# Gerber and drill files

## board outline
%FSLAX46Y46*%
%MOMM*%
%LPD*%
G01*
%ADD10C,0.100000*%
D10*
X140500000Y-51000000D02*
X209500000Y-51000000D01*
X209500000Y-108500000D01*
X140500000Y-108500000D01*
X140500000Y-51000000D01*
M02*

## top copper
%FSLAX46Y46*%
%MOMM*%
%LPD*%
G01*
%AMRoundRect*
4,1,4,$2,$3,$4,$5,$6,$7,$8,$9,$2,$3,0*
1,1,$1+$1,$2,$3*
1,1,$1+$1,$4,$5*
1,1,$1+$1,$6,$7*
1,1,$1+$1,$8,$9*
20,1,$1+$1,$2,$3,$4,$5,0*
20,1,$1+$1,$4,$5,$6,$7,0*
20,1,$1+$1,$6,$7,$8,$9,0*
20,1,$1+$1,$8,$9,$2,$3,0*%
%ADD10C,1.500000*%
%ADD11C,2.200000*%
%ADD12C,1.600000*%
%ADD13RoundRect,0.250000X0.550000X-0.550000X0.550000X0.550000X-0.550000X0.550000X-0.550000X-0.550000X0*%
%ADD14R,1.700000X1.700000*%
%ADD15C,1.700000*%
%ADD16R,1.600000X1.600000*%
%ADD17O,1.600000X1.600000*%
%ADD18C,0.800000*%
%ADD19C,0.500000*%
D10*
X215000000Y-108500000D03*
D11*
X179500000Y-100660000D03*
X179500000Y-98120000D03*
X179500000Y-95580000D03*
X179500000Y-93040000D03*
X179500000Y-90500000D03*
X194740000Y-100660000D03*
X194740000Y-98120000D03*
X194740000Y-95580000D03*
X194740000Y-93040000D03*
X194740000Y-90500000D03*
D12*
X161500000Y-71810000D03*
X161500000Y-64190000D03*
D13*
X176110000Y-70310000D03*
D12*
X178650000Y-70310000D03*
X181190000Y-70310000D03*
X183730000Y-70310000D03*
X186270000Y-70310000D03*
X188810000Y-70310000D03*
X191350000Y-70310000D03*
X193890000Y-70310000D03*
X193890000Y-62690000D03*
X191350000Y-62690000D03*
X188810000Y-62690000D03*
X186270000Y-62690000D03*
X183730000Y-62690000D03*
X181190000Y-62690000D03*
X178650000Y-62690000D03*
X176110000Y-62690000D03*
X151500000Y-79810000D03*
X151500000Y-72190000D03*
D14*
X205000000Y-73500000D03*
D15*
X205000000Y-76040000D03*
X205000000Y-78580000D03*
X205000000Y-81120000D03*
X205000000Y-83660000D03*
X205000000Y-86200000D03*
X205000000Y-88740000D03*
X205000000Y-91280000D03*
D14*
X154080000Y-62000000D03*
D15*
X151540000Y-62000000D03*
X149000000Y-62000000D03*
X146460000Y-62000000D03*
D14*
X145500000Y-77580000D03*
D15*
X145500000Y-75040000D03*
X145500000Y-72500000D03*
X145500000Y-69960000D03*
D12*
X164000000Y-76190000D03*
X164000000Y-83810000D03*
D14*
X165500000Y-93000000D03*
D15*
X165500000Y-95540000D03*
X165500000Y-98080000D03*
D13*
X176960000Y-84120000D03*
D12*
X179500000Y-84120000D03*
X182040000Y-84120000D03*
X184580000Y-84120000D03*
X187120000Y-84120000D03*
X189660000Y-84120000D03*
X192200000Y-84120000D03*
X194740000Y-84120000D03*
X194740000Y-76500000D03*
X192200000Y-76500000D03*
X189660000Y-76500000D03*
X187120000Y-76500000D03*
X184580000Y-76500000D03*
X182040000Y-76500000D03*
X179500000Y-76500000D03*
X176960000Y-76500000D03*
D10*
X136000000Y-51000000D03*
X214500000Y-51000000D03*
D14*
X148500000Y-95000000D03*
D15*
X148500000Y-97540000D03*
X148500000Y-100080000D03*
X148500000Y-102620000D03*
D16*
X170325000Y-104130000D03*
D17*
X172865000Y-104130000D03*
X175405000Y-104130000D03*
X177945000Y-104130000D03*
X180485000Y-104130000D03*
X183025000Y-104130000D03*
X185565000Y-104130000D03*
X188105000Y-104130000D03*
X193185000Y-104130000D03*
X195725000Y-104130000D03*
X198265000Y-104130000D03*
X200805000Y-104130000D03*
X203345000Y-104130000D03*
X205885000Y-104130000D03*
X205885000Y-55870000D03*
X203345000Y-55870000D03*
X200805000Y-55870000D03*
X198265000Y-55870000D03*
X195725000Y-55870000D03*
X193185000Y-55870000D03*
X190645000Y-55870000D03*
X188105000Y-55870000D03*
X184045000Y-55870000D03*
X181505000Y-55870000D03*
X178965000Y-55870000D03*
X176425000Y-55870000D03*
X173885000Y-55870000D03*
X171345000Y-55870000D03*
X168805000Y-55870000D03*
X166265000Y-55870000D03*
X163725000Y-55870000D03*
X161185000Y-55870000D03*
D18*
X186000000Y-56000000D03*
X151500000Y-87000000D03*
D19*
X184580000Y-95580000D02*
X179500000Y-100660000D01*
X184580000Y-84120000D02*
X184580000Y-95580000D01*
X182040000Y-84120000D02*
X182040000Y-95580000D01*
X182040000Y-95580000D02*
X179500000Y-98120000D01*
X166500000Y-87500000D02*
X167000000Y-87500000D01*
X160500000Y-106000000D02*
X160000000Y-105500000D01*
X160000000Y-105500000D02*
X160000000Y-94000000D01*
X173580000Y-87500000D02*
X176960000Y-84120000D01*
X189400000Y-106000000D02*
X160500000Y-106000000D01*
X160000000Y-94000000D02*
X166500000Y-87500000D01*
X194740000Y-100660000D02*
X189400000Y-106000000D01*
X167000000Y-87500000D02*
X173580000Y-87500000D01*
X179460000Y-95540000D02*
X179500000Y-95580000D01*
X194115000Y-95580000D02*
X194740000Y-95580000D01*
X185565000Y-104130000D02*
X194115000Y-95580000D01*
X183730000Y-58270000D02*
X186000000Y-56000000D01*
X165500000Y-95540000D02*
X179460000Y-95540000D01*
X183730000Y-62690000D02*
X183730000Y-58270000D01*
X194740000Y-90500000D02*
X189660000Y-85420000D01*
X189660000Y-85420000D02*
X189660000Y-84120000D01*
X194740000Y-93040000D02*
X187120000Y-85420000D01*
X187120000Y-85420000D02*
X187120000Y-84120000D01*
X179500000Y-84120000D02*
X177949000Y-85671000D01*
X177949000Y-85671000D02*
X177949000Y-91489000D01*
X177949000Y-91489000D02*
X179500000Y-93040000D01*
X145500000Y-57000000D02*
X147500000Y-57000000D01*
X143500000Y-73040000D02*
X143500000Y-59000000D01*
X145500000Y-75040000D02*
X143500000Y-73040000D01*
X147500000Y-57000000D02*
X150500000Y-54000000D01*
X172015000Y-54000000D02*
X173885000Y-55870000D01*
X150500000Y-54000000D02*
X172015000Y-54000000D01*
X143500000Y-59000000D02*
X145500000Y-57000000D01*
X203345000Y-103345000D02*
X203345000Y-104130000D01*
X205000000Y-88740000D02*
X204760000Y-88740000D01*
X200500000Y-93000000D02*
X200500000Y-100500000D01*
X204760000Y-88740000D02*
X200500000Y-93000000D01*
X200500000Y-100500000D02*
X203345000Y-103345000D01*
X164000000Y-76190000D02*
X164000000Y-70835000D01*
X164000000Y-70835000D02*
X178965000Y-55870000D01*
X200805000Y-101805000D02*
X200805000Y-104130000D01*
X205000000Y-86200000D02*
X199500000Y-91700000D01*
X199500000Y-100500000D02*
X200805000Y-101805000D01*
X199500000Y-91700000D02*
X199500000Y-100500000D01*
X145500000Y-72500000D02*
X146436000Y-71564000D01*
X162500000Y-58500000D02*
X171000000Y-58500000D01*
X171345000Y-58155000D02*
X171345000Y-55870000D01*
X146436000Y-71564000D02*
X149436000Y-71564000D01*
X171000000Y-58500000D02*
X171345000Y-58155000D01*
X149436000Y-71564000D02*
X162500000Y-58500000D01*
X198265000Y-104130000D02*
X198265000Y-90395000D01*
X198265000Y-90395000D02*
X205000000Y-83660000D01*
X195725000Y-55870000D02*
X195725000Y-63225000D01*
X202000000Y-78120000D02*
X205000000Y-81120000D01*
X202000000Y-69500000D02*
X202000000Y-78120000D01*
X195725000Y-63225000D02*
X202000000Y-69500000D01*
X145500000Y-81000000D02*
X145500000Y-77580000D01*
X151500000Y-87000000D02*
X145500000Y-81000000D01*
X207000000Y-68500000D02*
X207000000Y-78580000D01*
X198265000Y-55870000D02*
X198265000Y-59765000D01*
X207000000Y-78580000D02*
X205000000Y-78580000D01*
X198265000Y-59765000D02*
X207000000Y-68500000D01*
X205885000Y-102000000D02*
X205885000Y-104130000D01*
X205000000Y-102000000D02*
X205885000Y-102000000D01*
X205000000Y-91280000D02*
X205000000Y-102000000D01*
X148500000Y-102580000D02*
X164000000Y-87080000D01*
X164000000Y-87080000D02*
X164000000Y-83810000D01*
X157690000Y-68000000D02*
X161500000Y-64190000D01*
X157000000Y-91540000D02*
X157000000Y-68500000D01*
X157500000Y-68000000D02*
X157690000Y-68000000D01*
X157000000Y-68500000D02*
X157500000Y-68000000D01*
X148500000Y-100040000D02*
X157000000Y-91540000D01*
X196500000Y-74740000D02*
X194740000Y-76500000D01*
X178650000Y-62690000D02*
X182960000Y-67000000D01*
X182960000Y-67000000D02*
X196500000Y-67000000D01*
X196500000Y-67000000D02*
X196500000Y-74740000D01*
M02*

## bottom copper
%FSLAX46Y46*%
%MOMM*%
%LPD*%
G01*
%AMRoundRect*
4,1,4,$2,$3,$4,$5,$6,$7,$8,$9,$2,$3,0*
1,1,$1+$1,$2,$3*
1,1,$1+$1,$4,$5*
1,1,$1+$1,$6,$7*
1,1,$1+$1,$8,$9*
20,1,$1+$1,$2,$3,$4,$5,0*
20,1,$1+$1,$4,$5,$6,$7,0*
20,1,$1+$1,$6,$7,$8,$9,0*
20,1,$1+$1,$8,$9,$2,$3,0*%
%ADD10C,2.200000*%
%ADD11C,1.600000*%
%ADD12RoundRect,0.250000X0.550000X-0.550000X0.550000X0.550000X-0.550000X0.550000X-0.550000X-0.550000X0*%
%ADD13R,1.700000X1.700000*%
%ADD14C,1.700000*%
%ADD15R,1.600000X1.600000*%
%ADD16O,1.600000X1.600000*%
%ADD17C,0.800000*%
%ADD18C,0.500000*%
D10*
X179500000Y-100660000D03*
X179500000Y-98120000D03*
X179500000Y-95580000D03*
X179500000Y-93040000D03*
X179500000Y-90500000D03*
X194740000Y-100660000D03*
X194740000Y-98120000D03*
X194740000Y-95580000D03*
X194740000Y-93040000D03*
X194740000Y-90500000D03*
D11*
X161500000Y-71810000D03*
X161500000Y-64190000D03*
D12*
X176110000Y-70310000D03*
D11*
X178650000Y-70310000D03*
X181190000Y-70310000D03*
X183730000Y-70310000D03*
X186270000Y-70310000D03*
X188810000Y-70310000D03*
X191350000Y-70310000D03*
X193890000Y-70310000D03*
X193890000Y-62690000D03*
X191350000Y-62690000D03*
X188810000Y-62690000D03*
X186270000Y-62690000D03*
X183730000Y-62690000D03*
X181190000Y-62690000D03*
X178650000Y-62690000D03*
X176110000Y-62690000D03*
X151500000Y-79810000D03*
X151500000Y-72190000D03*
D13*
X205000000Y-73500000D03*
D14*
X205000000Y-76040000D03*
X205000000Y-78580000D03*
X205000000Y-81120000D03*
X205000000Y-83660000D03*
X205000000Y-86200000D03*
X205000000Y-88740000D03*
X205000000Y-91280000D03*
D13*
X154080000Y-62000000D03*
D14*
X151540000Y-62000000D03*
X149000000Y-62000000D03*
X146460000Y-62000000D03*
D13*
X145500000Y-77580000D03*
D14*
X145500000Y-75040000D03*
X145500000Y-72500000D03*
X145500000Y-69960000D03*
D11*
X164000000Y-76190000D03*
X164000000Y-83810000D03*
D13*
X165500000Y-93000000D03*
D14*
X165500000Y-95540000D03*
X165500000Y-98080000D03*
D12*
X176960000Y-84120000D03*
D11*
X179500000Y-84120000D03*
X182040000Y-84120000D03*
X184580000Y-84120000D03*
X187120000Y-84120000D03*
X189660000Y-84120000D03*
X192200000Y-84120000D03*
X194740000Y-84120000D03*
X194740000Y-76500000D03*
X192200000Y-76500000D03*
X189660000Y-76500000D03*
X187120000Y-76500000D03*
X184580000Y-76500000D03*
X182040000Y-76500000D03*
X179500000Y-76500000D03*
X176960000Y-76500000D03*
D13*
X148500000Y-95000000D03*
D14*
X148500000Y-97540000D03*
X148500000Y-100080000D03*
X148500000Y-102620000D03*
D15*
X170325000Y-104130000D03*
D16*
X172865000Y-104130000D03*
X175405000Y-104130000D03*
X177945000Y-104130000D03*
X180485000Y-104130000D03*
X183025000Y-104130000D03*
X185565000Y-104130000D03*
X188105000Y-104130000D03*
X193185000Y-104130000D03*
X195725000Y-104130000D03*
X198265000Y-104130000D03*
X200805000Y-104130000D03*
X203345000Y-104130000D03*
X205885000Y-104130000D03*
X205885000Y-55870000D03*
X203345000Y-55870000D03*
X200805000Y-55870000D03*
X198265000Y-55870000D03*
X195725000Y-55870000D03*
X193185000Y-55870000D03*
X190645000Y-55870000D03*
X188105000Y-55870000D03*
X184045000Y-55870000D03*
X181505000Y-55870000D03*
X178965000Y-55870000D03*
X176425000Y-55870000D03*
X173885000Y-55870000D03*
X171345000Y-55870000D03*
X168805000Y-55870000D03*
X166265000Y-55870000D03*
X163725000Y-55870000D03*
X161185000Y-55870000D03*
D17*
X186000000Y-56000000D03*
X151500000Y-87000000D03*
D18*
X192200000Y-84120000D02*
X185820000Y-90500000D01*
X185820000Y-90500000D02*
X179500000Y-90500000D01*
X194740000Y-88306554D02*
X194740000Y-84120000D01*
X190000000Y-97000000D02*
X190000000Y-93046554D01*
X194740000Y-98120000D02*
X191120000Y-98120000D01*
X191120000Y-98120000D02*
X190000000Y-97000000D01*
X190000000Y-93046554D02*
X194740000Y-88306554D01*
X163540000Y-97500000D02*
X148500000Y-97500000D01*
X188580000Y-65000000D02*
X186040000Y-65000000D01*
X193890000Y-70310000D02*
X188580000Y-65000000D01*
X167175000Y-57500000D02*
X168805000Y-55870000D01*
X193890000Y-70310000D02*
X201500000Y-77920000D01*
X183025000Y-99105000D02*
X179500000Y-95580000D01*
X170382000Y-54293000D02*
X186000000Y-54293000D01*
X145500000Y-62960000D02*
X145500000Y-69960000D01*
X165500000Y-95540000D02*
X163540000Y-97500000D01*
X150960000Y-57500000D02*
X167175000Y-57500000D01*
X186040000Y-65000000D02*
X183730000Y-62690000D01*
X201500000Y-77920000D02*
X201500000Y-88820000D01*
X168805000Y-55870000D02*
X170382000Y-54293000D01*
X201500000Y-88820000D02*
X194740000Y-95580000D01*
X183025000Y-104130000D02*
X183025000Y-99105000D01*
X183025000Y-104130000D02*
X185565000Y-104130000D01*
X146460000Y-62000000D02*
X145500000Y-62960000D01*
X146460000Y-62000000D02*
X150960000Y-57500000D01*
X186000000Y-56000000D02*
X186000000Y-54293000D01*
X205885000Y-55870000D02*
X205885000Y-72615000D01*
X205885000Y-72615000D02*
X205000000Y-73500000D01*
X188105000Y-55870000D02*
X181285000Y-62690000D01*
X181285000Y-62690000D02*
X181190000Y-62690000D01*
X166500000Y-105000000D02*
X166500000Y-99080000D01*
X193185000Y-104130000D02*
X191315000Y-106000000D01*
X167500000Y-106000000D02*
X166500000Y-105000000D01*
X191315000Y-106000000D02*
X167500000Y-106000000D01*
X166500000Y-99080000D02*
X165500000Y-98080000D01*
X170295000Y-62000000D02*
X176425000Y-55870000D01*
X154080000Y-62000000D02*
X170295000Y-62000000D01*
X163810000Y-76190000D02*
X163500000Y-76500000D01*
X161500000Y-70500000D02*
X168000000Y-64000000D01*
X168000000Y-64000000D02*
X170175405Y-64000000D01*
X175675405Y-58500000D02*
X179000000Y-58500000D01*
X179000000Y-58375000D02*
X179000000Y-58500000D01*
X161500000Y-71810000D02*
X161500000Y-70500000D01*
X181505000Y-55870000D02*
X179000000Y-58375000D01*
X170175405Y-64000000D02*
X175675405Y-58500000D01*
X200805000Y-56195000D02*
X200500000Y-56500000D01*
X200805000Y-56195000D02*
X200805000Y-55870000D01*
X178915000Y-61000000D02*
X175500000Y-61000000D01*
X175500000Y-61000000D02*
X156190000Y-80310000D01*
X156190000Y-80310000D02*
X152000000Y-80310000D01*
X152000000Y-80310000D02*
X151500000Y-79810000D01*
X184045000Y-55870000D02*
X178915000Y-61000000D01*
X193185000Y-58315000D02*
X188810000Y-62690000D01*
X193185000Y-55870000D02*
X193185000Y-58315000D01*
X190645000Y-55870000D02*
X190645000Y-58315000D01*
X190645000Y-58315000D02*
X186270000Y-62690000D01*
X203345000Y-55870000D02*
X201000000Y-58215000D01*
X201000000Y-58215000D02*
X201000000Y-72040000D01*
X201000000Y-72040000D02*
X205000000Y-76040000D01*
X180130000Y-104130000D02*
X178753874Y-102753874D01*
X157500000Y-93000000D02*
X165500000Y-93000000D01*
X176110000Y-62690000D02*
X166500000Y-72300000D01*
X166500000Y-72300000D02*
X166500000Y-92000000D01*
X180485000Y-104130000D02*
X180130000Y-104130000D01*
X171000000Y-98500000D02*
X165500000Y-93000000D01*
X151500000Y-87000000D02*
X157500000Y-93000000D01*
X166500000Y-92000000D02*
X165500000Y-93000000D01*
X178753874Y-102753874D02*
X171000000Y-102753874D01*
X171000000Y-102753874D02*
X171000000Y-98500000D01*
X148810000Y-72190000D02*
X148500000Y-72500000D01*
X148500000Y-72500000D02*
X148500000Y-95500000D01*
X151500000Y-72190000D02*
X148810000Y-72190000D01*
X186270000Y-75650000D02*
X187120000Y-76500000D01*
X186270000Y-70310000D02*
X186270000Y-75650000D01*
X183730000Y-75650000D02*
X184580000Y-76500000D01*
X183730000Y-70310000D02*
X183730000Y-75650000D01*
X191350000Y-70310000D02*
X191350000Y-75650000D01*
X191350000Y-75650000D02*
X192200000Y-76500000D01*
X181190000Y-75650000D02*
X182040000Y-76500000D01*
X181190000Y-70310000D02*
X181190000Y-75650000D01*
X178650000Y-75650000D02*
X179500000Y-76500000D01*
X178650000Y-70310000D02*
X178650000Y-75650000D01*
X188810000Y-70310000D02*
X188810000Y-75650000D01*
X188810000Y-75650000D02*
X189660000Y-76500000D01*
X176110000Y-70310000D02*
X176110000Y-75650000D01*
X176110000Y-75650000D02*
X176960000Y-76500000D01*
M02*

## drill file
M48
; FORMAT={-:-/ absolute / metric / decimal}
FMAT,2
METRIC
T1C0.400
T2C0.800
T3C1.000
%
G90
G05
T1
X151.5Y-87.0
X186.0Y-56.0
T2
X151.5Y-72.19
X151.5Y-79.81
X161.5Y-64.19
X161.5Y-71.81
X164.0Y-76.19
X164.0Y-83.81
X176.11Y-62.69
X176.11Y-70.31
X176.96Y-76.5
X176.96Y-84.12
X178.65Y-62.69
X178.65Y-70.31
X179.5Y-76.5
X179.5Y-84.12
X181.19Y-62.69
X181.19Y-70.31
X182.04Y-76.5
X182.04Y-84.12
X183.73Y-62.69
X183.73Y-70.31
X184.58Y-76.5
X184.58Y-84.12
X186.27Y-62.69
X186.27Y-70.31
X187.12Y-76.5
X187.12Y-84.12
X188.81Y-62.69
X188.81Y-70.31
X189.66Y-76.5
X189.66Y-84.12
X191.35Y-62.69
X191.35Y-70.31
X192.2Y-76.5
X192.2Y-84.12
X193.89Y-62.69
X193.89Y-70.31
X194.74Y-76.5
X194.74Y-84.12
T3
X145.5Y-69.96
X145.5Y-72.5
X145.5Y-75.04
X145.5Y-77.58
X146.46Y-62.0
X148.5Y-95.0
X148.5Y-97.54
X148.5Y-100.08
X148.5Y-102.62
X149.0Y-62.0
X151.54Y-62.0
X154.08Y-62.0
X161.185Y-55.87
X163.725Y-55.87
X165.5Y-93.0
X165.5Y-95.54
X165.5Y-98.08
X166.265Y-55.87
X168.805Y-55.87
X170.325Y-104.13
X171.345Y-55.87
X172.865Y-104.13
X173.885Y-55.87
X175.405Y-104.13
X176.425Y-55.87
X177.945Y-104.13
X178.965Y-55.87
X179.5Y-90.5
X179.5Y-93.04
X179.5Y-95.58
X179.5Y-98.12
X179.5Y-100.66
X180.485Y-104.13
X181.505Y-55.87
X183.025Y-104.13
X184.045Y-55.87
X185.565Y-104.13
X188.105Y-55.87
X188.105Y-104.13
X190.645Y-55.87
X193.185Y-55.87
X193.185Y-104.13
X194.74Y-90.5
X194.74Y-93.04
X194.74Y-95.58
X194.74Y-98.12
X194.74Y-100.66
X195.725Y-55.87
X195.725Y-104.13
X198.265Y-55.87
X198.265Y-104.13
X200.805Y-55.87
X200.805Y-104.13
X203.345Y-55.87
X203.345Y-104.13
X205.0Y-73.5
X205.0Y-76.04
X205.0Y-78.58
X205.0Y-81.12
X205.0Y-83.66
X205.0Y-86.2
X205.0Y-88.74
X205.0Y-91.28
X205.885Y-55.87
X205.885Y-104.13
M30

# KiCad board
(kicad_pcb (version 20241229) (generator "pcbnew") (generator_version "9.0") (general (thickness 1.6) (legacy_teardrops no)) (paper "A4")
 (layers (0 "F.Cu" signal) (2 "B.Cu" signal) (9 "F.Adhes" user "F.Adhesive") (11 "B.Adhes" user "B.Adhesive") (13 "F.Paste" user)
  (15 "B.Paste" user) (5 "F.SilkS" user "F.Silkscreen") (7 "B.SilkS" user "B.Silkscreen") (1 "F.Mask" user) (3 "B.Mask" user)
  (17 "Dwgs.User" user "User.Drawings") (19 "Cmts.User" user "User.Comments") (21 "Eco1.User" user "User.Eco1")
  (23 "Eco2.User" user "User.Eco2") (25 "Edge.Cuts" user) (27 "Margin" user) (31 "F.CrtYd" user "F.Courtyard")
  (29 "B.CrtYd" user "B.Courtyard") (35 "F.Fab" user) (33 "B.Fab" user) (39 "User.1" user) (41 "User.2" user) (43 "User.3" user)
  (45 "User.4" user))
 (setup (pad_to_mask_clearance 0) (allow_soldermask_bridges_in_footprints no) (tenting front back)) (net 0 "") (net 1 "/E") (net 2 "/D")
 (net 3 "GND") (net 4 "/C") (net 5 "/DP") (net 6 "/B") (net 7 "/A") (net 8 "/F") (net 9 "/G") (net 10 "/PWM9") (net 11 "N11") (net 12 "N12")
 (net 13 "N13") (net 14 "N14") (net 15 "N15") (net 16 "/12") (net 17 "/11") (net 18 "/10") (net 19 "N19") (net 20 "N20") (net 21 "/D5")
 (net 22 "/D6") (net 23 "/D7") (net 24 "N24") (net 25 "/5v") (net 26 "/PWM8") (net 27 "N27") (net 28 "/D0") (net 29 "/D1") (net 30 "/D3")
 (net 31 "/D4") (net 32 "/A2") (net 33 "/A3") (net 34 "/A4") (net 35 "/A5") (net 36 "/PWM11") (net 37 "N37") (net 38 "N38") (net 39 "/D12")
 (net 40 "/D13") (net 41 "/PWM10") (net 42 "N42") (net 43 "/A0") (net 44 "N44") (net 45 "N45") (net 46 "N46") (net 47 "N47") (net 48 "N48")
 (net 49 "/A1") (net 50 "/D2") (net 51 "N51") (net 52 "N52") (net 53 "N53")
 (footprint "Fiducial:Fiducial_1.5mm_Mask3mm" (layer "F.Cu") (at 215 108.5)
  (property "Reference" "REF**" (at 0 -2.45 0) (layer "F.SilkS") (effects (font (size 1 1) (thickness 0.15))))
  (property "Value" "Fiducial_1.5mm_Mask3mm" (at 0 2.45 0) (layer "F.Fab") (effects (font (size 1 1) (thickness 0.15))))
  (pad "" smd circle (at 0 0) (size 1.5 1.5) (layers "F.Cu" "F.Mask") (solder_mask_margin 0.75)))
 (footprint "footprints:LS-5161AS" (layer "F.Cu") (at 179.5 100.66 90)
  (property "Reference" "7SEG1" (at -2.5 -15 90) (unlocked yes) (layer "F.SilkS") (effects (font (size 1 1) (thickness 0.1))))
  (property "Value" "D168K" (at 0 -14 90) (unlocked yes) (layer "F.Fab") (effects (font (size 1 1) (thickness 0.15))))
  (pad "1" thru_hole circle (at 0 0 90) (size 2.2 2.2) (drill 1) (layers "*.Cu" "*.Mask") (remove_unused_layers no) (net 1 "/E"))
  (pad "2" thru_hole circle (at 2.54 0 90) (size 2.2 2.2) (drill 1) (layers "*.Cu" "*.Mask") (remove_unused_layers no) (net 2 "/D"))
  (pad "3" thru_hole circle (at 5.08 0 90) (size 2.2 2.2) (drill 1) (layers "*.Cu" "*.Mask") (remove_unused_layers no) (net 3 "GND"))
  (pad "4" thru_hole circle (at 7.62 0 90) (size 2.2 2.2) (drill 1) (layers "*.Cu" "*.Mask") (remove_unused_layers no) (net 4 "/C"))
  (pad "5" thru_hole circle (at 10.16 0 90) (size 2.2 2.2) (drill 1) (layers "*.Cu" "*.Mask") (remove_unused_layers no) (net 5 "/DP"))
  (pad "6" thru_hole circle (at 0 15.24 90) (size 2.2 2.2) (drill 1) (layers "*.Cu" "*.Mask") (remove_unused_layers no) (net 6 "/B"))
  (pad "7" thru_hole circle (at 2.54 15.24 90) (size 2.2 2.2) (drill 1) (layers "*.Cu" "*.Mask") (remove_unused_layers no) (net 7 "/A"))
  (pad "8" thru_hole circle (at 5.08 15.24 90) (size 2.2 2.2) (drill 1) (layers "*.Cu" "*.Mask") (remove_unused_layers no) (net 3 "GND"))
  (pad "9" thru_hole circle (at 7.62 15.24 90) (size 2.2 2.2) (drill 1) (layers "*.Cu" "*.Mask") (remove_unused_layers no) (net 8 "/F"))
  (pad "10" thru_hole circle (at 10.16 15.24 90) (size 2.2 2.2) (drill 1) (layers "*.Cu" "*.Mask") (remove_unused_layers no) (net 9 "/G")))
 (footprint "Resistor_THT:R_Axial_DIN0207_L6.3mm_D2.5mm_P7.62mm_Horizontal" (layer "F.Cu") (at 161.5 71.81 90)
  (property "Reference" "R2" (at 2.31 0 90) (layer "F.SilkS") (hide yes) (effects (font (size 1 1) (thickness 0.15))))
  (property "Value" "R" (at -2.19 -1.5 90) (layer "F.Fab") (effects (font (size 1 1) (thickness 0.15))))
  (pad "1" thru_hole circle (at 0 0 90) (size 1.6 1.6) (drill 0.8) (layers "*.Cu" "*.Mask") (remove_unused_layers no) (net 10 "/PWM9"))
  (pad "2" thru_hole circle (at 7.62 0 90) (size 1.6 1.6) (drill 0.8) (layers "*.Cu" "*.Mask") (remove_unused_layers no) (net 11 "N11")))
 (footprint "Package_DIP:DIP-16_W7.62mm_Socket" (layer "F.Cu") (at 176.11 70.31 90)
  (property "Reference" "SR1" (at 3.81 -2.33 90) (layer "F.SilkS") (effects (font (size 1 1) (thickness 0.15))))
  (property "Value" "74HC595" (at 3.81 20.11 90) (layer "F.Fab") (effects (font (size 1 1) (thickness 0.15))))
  (pad "1" thru_hole roundrect (at 0 0 90) (size 1.6 1.6) (drill 0.8) (layers "*.Cu" "*.Mask") (remove_unused_layers no)
   (roundrect_rratio 0.15625) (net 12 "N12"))
  (pad "2" thru_hole circle (at 0 2.54 90) (size 1.6 1.6) (drill 0.8) (layers "*.Cu" "*.Mask") (remove_unused_layers no) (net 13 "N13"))
  (pad "3" thru_hole circle (at 0 5.08 90) (size 1.6 1.6) (drill 0.8) (layers "*.Cu" "*.Mask") (remove_unused_layers no) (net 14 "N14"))
  (pad "4" thru_hole circle (at 0 7.62 90) (size 1.6 1.6) (drill 0.8) (layers "*.Cu" "*.Mask") (remove_unused_layers no) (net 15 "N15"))
  (pad "5" thru_hole circle (at 0 10.16 90) (size 1.6 1.6) (drill 0.8) (layers "*.Cu" "*.Mask") (remove_unused_layers no) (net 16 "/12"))
  (pad "6" thru_hole circle (at 0 12.7 90) (size 1.6 1.6) (drill 0.8) (layers "*.Cu" "*.Mask") (remove_unused_layers no) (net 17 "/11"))
  (pad "7" thru_hole circle (at 0 15.24 90) (size 1.6 1.6) (drill 0.8) (layers "*.Cu" "*.Mask") (remove_unused_layers no) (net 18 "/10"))
  (pad "8" thru_hole circle (at 0 17.78 90) (size 1.6 1.6) (drill 0.8) (layers "*.Cu" "*.Mask") (remove_unused_layers no) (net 3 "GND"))
  (pad "9" thru_hole circle (at 7.62 17.78 90) (size 1.6 1.6) (drill 0.8) (layers "*.Cu" "*.Mask") (remove_unused_layers no) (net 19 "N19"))
  (pad "10" thru_hole circle (at 7.62 15.24 90) (size 1.6 1.6) (drill 0.8) (layers "*.Cu" "*.Mask") (remove_unused_layers no) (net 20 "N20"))
  (pad "11" thru_hole circle (at 7.62 12.7 90) (size 1.6 1.6) (drill 0.8) (layers "*.Cu" "*.Mask") (remove_unused_layers no) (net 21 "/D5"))
  (pad "12" thru_hole circle (at 7.62 10.16 90) (size 1.6 1.6) (drill 0.8) (layers "*.Cu" "*.Mask") (remove_unused_layers no) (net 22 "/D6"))
  (pad "13" thru_hole circle (at 7.62 7.62 90) (size 1.6 1.6) (drill 0.8) (layers "*.Cu" "*.Mask") (remove_unused_layers no) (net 3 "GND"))
  (pad "14" thru_hole circle (at 7.62 5.08 90) (size 1.6 1.6) (drill 0.8) (layers "*.Cu" "*.Mask") (remove_unused_layers no) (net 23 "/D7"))
  (pad "15" thru_hole circle (at 7.62 2.54 90) (size 1.6 1.6) (drill 0.8) (layers "*.Cu" "*.Mask") (remove_unused_layers no) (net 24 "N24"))
  (pad "16" thru_hole circle (at 7.62 0 90) (size 1.6 1.6) (drill 0.8) (layers "*.Cu" "*.Mask") (remove_unused_layers no) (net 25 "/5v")))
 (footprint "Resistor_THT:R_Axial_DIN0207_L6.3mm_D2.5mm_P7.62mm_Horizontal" (layer "F.Cu") (at 151.5 79.81 90)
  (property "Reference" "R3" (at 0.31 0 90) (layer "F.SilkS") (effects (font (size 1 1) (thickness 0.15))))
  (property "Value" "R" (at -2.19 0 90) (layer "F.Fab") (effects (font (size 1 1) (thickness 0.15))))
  (pad "1" thru_hole circle (at 0 0 90) (size 1.6 1.6) (drill 0.8) (layers "*.Cu" "*.Mask") (remove_unused_layers no) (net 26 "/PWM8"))
  (pad "2" thru_hole circle (at 7.62 0 90) (size 1.6 1.6) (drill 0.8) (layers "*.Cu" "*.Mask") (remove_unused_layers no) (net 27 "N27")))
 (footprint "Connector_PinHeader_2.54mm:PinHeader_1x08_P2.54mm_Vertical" (layer "F.Cu") (at 205 73.5)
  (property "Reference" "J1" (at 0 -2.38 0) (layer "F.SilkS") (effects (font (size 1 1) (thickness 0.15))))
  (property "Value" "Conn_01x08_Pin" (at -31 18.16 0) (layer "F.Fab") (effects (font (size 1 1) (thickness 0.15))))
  (pad "1" thru_hole rect (at 0 0) (size 1.7 1.7) (drill 1) (layers "*.Cu" "*.Mask") (remove_unused_layers no) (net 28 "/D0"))
  (pad "2" thru_hole circle (at 0 2.54) (size 1.7 1.7) (drill 1) (layers "*.Cu" "*.Mask") (remove_unused_layers no) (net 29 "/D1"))
  (pad "3" thru_hole circle (at 0 5.08) (size 1.7 1.7) (drill 1) (layers "*.Cu" "*.Mask") (remove_unused_layers no) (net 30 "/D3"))
  (pad "4" thru_hole circle (at 0 7.62) (size 1.7 1.7) (drill 1) (layers "*.Cu" "*.Mask") (remove_unused_layers no) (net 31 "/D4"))
  (pad "5" thru_hole circle (at 0 10.16) (size 1.7 1.7) (drill 1) (layers "*.Cu" "*.Mask") (remove_unused_layers no) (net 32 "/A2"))
  (pad "6" thru_hole circle (at 0 12.7) (size 1.7 1.7) (drill 1) (layers "*.Cu" "*.Mask") (remove_unused_layers no) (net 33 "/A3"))
  (pad "7" thru_hole circle (at 0 15.24) (size 1.7 1.7) (drill 1) (layers "*.Cu" "*.Mask") (remove_unused_layers no) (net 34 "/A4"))
  (pad "8" thru_hole circle (at 0 17.78) (size 1.7 1.7) (drill 1) (layers "*.Cu" "*.Mask") (remove_unused_layers no) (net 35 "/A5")))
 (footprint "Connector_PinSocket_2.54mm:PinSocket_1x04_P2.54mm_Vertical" (layer "F.Cu") (at 154.08 62 -90)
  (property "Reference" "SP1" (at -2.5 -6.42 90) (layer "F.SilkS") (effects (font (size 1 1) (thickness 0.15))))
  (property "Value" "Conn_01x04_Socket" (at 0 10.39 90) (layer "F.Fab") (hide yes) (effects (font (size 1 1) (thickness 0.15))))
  (pad "1" thru_hole rect (at 0 0 270) (size 1.7 1.7) (drill 1) (layers "*.Cu" "*.Mask") (remove_unused_layers no) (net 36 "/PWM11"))
  (pad "2" thru_hole circle (at 0 2.54 270) (size 1.7 1.7) (drill 1) (layers "*.Cu" "*.Mask") (remove_unused_layers no) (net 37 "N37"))
  (pad "3" thru_hole circle (at 0 5.08 270) (size 1.7 1.7) (drill 1) (layers "*.Cu" "*.Mask") (remove_unused_layers no) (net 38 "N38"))
  (pad "4" thru_hole circle (at 0 7.62 270) (size 1.7 1.7) (drill 1) (layers "*.Cu" "*.Mask") (remove_unused_layers no) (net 3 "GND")))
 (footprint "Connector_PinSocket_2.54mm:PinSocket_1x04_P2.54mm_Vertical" (layer "F.Cu") (at 145.5 77.58 180)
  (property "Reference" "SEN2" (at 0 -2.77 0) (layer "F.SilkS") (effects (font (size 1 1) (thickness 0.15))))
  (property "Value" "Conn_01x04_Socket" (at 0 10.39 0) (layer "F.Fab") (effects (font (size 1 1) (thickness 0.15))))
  (pad "1" thru_hole rect (at 0 0 180) (size 1.7 1.7) (drill 1) (layers "*.Cu" "*.Mask") (remove_unused_layers no) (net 25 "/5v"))
  (pad "2" thru_hole circle (at 0 2.54 180) (size 1.7 1.7) (drill 1) (layers "*.Cu" "*.Mask") (remove_unused_layers no) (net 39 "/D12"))
  (pad "3" thru_hole circle (at 0 5.08 180) (size 1.7 1.7) (drill 1) (layers "*.Cu" "*.Mask") (remove_unused_layers no) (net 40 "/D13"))
  (pad "4" thru_hole circle (at 0 7.62 180) (size 1.7 1.7) (drill 1) (layers "*.Cu" "*.Mask") (remove_unused_layers no) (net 3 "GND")))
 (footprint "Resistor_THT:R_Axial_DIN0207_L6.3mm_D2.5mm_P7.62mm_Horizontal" (layer "F.Cu") (at 164 76.19 -90)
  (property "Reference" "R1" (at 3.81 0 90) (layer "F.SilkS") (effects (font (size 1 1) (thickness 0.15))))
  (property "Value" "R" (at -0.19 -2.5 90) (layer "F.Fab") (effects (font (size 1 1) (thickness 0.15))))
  (pad "1" thru_hole circle (at 0 0 270) (size 1.6 1.6) (drill 0.8) (layers "*.Cu" "*.Mask") (remove_unused_layers no) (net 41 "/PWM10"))
  (pad "2" thru_hole circle (at 7.62 0 270) (size 1.6 1.6) (drill 0.8) (layers "*.Cu" "*.Mask") (remove_unused_layers no) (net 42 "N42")))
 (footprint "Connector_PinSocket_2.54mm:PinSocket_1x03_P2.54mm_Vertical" (layer "F.Cu") (at 165.5 93)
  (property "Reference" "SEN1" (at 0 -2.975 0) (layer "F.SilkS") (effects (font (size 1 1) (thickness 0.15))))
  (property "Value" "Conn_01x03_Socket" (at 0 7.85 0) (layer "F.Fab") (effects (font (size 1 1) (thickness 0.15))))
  (pad "1" thru_hole rect (at 0 0) (size 1.7 1.7) (drill 1) (layers "*.Cu" "*.Mask") (remove_unused_layers no) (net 25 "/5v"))
  (pad "2" thru_hole circle (at 0 2.54) (size 1.7 1.7) (drill 1) (layers "*.Cu" "*.Mask") (remove_unused_layers no) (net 3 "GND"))
  (pad "3" thru_hole circle (at 0 5.08) (size 1.7 1.7) (drill 1) (layers "*.Cu" "*.Mask") (remove_unused_layers no) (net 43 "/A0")))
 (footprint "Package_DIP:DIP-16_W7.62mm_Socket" (layer "F.Cu") (at 176.96 84.12 90)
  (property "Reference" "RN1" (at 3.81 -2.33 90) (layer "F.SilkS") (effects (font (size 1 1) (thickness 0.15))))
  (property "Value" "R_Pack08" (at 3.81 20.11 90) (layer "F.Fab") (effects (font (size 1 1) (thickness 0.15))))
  (pad "1" thru_hole roundrect (at 0 0 90) (size 1.6 1.6) (drill 0.8) (layers "*.Cu" "*.Mask") (remove_unused_layers no)
   (roundrect_rratio 0.15625) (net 6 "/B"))
  (pad "2" thru_hole circle (at 0 2.54 90) (size 1.6 1.6) (drill 0.8) (layers "*.Cu" "*.Mask") (remove_unused_layers no) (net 4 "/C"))
  (pad "3" thru_hole circle (at 0 5.08 90) (size 1.6 1.6) (drill 0.8) (layers "*.Cu" "*.Mask") (remove_unused_layers no) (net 2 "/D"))
  (pad "4" thru_hole circle (at 0 7.62 90) (size 1.6 1.6) (drill 0.8) (layers "*.Cu" "*.Mask") (remove_unused_layers no) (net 1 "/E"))
  (pad "5" thru_hole circle (at 0 10.16 90) (size 1.6 1.6) (drill 0.8) (layers "*.Cu" "*.Mask") (remove_unused_layers no) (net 8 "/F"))
  (pad "6" thru_hole circle (at 0 12.7 90) (size 1.6 1.6) (drill 0.8) (layers "*.Cu" "*.Mask") (remove_unused_layers no) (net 9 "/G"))
  (pad "7" thru_hole circle (at 0 15.24 90) (size 1.6 1.6) (drill 0.8) (layers "*.Cu" "*.Mask") (remove_unused_layers no) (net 5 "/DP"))
  (pad "8" thru_hole circle (at 0 17.78 90) (size 1.6 1.6) (drill 0.8) (layers "*.Cu" "*.Mask") (remove_unused_layers no) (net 7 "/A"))
  (pad "9" thru_hole circle (at 7.62 17.78 90) (size 1.6 1.6) (drill 0.8) (layers "*.Cu" "*.Mask") (remove_unused_layers no) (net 24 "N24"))
  (pad "10" thru_hole circle (at 7.62 15.24 90) (size 1.6 1.6) (drill 0.8) (layers "*.Cu" "*.Mask") (remove_unused_layers no) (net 18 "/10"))
  (pad "11" thru_hole circle (at 7.62 12.7 90) (size 1.6 1.6) (drill 0.8) (layers "*.Cu" "*.Mask") (remove_unused_layers no) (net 17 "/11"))
  (pad "12" thru_hole circle (at 7.62 10.16 90) (size 1.6 1.6) (drill 0.8) (layers "*.Cu" "*.Mask") (remove_unused_layers no) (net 16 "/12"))
  (pad "13" thru_hole circle (at 7.62 7.62 90) (size 1.6 1.6) (drill 0.8) (layers "*.Cu" "*.Mask") (remove_unused_layers no) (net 15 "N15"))
  (pad "14" thru_hole circle (at 7.62 5.08 90) (size 1.6 1.6) (drill 0.8) (layers "*.Cu" "*.Mask") (remove_unused_layers no) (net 14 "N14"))
  (pad "15" thru_hole circle (at 7.62 2.54 90) (size 1.6 1.6) (drill 0.8) (layers "*.Cu" "*.Mask") (remove_unused_layers no) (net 13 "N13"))
  (pad "16" thru_hole circle (at 7.62 0 90) (size 1.6 1.6) (drill 0.8) (layers "*.Cu" "*.Mask") (remove_unused_layers no) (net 12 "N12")))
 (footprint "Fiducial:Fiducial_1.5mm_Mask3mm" (layer "F.Cu") (at 136 51)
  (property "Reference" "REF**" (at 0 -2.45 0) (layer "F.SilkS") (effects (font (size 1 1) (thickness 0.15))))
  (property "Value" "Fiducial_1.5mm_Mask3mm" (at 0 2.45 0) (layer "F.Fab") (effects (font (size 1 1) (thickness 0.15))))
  (pad "" smd circle (at 0 0) (size 1.5 1.5) (layers "F.Cu" "F.Mask") (solder_mask_margin 0.75)))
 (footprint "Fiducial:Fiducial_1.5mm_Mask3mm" (layer "F.Cu") (at 214.5 51)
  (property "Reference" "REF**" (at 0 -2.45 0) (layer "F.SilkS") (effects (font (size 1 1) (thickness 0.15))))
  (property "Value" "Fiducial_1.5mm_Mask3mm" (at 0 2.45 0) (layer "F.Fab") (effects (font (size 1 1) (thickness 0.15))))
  (pad "" smd circle (at 0 0) (size 1.5 1.5) (layers "F.Cu" "F.Mask") (solder_mask_margin 0.75)))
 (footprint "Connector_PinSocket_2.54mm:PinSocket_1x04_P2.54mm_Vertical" (layer "F.Cu") (at 148.5 95)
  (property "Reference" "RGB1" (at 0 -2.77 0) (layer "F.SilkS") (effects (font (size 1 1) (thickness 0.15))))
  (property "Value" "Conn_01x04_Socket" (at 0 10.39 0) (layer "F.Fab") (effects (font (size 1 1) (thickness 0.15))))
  (pad "1" thru_hole rect (at 0 0) (size 1.7 1.7) (drill 1) (layers "*.Cu" "*.Mask") (remove_unused_layers no) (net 27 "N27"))
  (pad "2" thru_hole circle (at 0 2.54) (size 1.7 1.7) (drill 1) (layers "*.Cu" "*.Mask") (remove_unused_layers no) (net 3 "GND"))
  (pad "3" thru_hole circle (at 0 5.08) (size 1.7 1.7) (drill 1) (layers "*.Cu" "*.Mask") (remove_unused_layers no) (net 11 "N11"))
  (pad "4" thru_hole circle (at 0 7.62) (size 1.7 1.7) (drill 1) (layers "*.Cu" "*.Mask") (remove_unused_layers no) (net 42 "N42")))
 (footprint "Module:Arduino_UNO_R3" (layer "B.Cu") (at 170.325 104.13)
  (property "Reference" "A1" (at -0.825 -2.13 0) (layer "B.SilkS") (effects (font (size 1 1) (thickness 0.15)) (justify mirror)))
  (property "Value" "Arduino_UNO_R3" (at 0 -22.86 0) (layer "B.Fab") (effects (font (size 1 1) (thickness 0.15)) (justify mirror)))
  (pad "1" thru_hole rect (at 0 0 270) (size 1.6 1.6) (drill 1) (layers "*.Cu" "*.Mask") (remove_unused_layers no) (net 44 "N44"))
  (pad "2" thru_hole oval (at 2.54 0 270) (size 1.6 1.6) (drill 1) (layers "*.Cu" "*.Mask") (remove_unused_layers no) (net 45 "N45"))
  (pad "3" thru_hole oval (at 5.08 0 270) (size 1.6 1.6) (drill 1) (layers "*.Cu" "*.Mask") (remove_unused_layers no) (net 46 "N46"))
  (pad "4" thru_hole oval (at 7.62 0 270) (size 1.6 1.6) (drill 1) (layers "*.Cu" "*.Mask") (remove_unused_layers no) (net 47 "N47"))
  (pad "5" thru_hole oval (at 10.16 0 270) (size 1.6 1.6) (drill 1) (layers "*.Cu" "*.Mask") (remove_unused_layers no) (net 25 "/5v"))
  (pad "6" thru_hole oval (at 12.7 0 270) (size 1.6 1.6) (drill 1) (layers "*.Cu" "*.Mask") (remove_unused_layers no) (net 3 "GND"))
  (pad "7" thru_hole oval (at 15.24 0 270) (size 1.6 1.6) (drill 1) (layers "*.Cu" "*.Mask") (remove_unused_layers no) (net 3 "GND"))
  (pad "8" thru_hole oval (at 17.78 0 270) (size 1.6 1.6) (drill 1) (layers "*.Cu" "*.Mask") (remove_unused_layers no) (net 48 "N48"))
  (pad "9" thru_hole oval (at 22.86 0 270) (size 1.6 1.6) (drill 1) (layers "*.Cu" "*.Mask") (remove_unused_layers no) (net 43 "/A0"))
  (pad "10" thru_hole oval (at 25.4 0 270) (size 1.6 1.6) (drill 1) (layers "*.Cu" "*.Mask") (remove_unused_layers no) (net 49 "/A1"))
  (pad "11" thru_hole oval (at 27.94 0 270) (size 1.6 1.6) (drill 1) (layers "*.Cu" "*.Mask") (remove_unused_layers no) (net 32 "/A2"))
  (pad "12" thru_hole oval (at 30.48 0 270) (size 1.6 1.6) (drill 1) (layers "*.Cu" "*.Mask") (remove_unused_layers no) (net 33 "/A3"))
  (pad "13" thru_hole oval (at 33.02 0 270) (size 1.6 1.6) (drill 1) (layers "*.Cu" "*.Mask") (remove_unused_layers no) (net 34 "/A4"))
  (pad "14" thru_hole oval (at 35.56 0 270) (size 1.6 1.6) (drill 1) (layers "*.Cu" "*.Mask") (remove_unused_layers no) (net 35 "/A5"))
  (pad "15" thru_hole oval (at 35.56 -48.26 270) (size 1.6 1.6) (drill 1) (layers "*.Cu" "*.Mask") (remove_unused_layers no) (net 28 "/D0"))
  (pad "16" thru_hole oval (at 33.02 -48.26 270) (size 1.6 1.6) (drill 1) (layers "*.Cu" "*.Mask") (remove_unused_layers no) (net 29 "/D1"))
  (pad "17" thru_hole oval (at 30.48 -48.26 270) (size 1.6 1.6) (drill 1) (layers "*.Cu" "*.Mask") (remove_unused_layers no) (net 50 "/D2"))
  (pad "18" thru_hole oval (at 27.94 -48.26 270) (size 1.6 1.6) (drill 1) (layers "*.Cu" "*.Mask") (remove_unused_layers no) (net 30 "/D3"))
  (pad "19" thru_hole oval (at 25.4 -48.26 270) (size 1.6 1.6) (drill 1) (layers "*.Cu" "*.Mask") (remove_unused_layers no) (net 31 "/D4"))
  (pad "20" thru_hole oval (at 22.86 -48.26 270) (size 1.6 1.6) (drill 1) (layers "*.Cu" "*.Mask") (remove_unused_layers no) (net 21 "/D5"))
  (pad "21" thru_hole oval (at 20.32 -48.26 270) (size 1.6 1.6) (drill 1) (layers "*.Cu" "*.Mask") (remove_unused_layers no) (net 22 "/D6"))
  (pad "22" thru_hole oval (at 17.78 -48.26 270) (size 1.6 1.6) (drill 1) (layers "*.Cu" "*.Mask") (remove_unused_layers no) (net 23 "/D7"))
  (pad "23" thru_hole oval (at 13.72 -48.26 270) (size 1.6 1.6) (drill 1) (layers "*.Cu" "*.Mask") (remove_unused_layers no)
   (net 26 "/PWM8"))
  (pad "24" thru_hole oval (at 11.18 -48.26 270) (size 1.6 1.6) (drill 1) (layers "*.Cu" "*.Mask") (remove_unused_layers no)
   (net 10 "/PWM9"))
  (pad "25" thru_hole oval (at 8.64 -48.26 270) (size 1.6 1.6) (drill 1) (layers "*.Cu" "*.Mask") (remove_unused_layers no)
   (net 41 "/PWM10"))
  (pad "26" thru_hole oval (at 6.1 -48.26 270) (size 1.6 1.6) (drill 1) (layers "*.Cu" "*.Mask") (remove_unused_layers no) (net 36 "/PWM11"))
  (pad "27" thru_hole oval (at 3.56 -48.26 270) (size 1.6 1.6) (drill 1) (layers "*.Cu" "*.Mask") (remove_unused_layers no) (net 39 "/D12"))
  (pad "28" thru_hole oval (at 1.02 -48.26 270) (size 1.6 1.6) (drill 1) (layers "*.Cu" "*.Mask") (remove_unused_layers no) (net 40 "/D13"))
  (pad "29" thru_hole oval (at -1.52 -48.26 270) (size 1.6 1.6) (drill 1) (layers "*.Cu" "*.Mask") (remove_unused_layers no) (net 3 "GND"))
  (pad "30" thru_hole oval (at -4.06 -48.26 270) (size 1.6 1.6) (drill 1) (layers "*.Cu" "*.Mask") (remove_unused_layers no) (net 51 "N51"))
  (pad "31" thru_hole oval (at -6.6 -48.26 270) (size 1.6 1.6) (drill 1) (layers "*.Cu" "*.Mask") (remove_unused_layers no) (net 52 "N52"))
  (pad "32" thru_hole oval (at -9.14 -48.26 270) (size 1.6 1.6) (drill 1) (layers "*.Cu" "*.Mask") (remove_unused_layers no) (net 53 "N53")))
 (gr_rect (start 140.5 51) (end 209.5 108.5) (stroke (width 0.1) (type default)) (fill no) (layer "Edge.Cuts"))
 (segment (start 184.58 95.58) (end 179.5 100.66) (width 0.5) (layer "F.Cu") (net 1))
 (segment (start 184.58 84.12) (end 184.58 95.58) (width 0.5) (layer "F.Cu") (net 1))
 (segment (start 182.04 84.12) (end 182.04 95.58) (width 0.5) (layer "F.Cu") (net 2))
 (segment (start 182.04 95.58) (end 179.5 98.12) (width 0.5) (layer "F.Cu") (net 2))
 (segment (start 192.2 84.12) (end 185.82 90.5) (width 0.5) (layer "B.Cu") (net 5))
 (segment (start 185.82 90.5) (end 179.5 90.5) (width 0.5) (layer "B.Cu") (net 5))
 (segment (start 166.5 87.5) (end 167 87.5) (width 0.5) (layer "F.Cu") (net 6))
 (segment (start 160.5 106) (end 160 105.5) (width 0.5) (layer "F.Cu") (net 6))
 (segment (start 160 105.5) (end 160 94) (width 0.5) (layer "F.Cu") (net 6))
 (segment (start 173.58 87.5) (end 176.96 84.12) (width 0.5) (layer "F.Cu") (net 6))
 (segment (start 189.4 106) (end 160.5 106) (width 0.5) (layer "F.Cu") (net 6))
 (segment (start 160 94) (end 166.5 87.5) (width 0.5) (layer "F.Cu") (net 6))
 (segment (start 194.74 100.66) (end 189.4 106) (width 0.5) (layer "F.Cu") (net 6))
 (segment (start 167 87.5) (end 173.58 87.5) (width 0.5) (layer "F.Cu") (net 6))
 (segment (start 194.74 88.306554) (end 194.74 84.12) (width 0.5) (layer "B.Cu") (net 7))
 (segment (start 190 97) (end 190 93.046554) (width 0.5) (layer "B.Cu") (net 7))
 (segment (start 194.74 98.12) (end 191.12 98.12) (width 0.5) (layer "B.Cu") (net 7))
 (segment (start 191.12 98.12) (end 190 97) (width 0.5) (layer "B.Cu") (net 7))
 (segment (start 190 93.046554) (end 194.74 88.306554) (width 0.5) (layer "B.Cu") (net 7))
 (segment (start 179.46 95.54) (end 179.5 95.58) (width 0.5) (layer "F.Cu") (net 3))
 (segment (start 194.115 95.58) (end 194.74 95.58) (width 0.5) (layer "F.Cu") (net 3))
 (segment (start 185.565 104.13) (end 194.115 95.58) (width 0.5) (layer "F.Cu") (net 3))
 (segment (start 183.73 58.27) (end 186 56) (width 0.5) (layer "F.Cu") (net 3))
 (segment (start 165.5 95.54) (end 179.46 95.54) (width 0.5) (layer "F.Cu") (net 3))
 (segment (start 183.73 62.69) (end 183.73 58.27) (width 0.5) (layer "F.Cu") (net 3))
 (via (at 186 56) (size 0.8) (drill 0.4) (layers "F.Cu" "B.Cu") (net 3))
 (segment (start 163.54 97.5) (end 148.5 97.5) (width 0.5) (layer "B.Cu") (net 3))
 (segment (start 188.58 65) (end 186.04 65) (width 0.5) (layer "B.Cu") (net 3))
 (segment (start 193.89 70.31) (end 188.58 65) (width 0.5) (layer "B.Cu") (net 3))
 (segment (start 167.175 57.5) (end 168.805 55.87) (width 0.5) (layer "B.Cu") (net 3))
 (segment (start 193.89 70.31) (end 201.5 77.92) (width 0.5) (layer "B.Cu") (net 3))
 (segment (start 183.025 99.105) (end 179.5 95.58) (width 0.5) (layer "B.Cu") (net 3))
 (segment (start 170.382 54.293) (end 186 54.293) (width 0.5) (layer "B.Cu") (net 3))
 (segment (start 145.5 62.96) (end 145.5 69.96) (width 0.5) (layer "B.Cu") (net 3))
 (segment (start 165.5 95.54) (end 163.54 97.5) (width 0.5) (layer "B.Cu") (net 3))
 (segment (start 150.96 57.5) (end 167.175 57.5) (width 0.5) (layer "B.Cu") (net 3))
 (segment (start 186.04 65) (end 183.73 62.69) (width 0.5) (layer "B.Cu") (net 3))
 (segment (start 201.5 77.92) (end 201.5 88.82) (width 0.5) (layer "B.Cu") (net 3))
 (segment (start 168.805 55.87) (end 170.382 54.293) (width 0.5) (layer "B.Cu") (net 3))
 (segment (start 201.5 88.82) (end 194.74 95.58) (width 0.5) (layer "B.Cu") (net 3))
 (segment (start 183.025 104.13) (end 183.025 99.105) (width 0.5) (layer "B.Cu") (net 3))
 (segment (start 183.025 104.13) (end 185.565 104.13) (width 0.5) (layer "B.Cu") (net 3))
 (segment (start 146.46 62) (end 145.5 62.96) (width 0.5) (layer "B.Cu") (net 3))
 (segment (start 146.46 62) (end 150.96 57.5) (width 0.5) (layer "B.Cu") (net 3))
 (segment (start 186 56) (end 186 54.293) (width 0.5) (layer "B.Cu") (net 3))
 (segment (start 194.74 90.5) (end 189.66 85.42) (width 0.5) (layer "F.Cu") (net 9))
 (segment (start 189.66 85.42) (end 189.66 84.12) (width 0.5) (layer "F.Cu") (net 9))
 (segment (start 194.74 93.04) (end 187.12 85.42) (width 0.5) (layer "F.Cu") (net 8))
 (segment (start 187.12 85.42) (end 187.12 84.12) (width 0.5) (layer "F.Cu") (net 8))
 (segment (start 179.5 84.12) (end 177.949 85.671) (width 0.5) (layer "F.Cu") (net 4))
 (segment (start 177.949 85.671) (end 177.949 91.489) (width 0.5) (layer "F.Cu") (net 4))
 (segment (start 177.949 91.489) (end 179.5 93.04) (width 0.5) (layer "F.Cu") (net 4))
 (segment (start 145.5 57) (end 147.5 57) (width 0.5) (layer "F.Cu") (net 39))
 (segment (start 143.5 73.04) (end 143.5 59) (width 0.5) (layer "F.Cu") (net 39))
 (segment (start 145.5 75.04) (end 143.5 73.04) (width 0.5) (layer "F.Cu") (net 39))
 (segment (start 147.5 57) (end 150.5 54) (width 0.5) (layer "F.Cu") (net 39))
 (segment (start 172.015 54) (end 173.885 55.87) (width 0.5) (layer "F.Cu") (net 39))
 (segment (start 150.5 54) (end 172.015 54) (width 0.5) (layer "F.Cu") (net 39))
 (segment (start 143.5 59) (end 145.5 57) (width 0.5) (layer "F.Cu") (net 39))
 (segment (start 205.885 55.87) (end 205.885 72.615) (width 0.5) (layer "B.Cu") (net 28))
 (segment (start 205.885 72.615) (end 205 73.5) (width 0.5) (layer "B.Cu") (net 28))
 (segment (start 203.345 103.345) (end 203.345 104.13) (width 0.5) (layer "F.Cu") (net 34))
 (segment (start 205 88.74) (end 204.76 88.74) (width 0.5) (layer "F.Cu") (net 34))
 (segment (start 200.5 93) (end 200.5 100.5) (width 0.5) (layer "F.Cu") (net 34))
 (segment (start 204.76 88.74) (end 200.5 93) (width 0.5) (layer "F.Cu") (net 34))
 (segment (start 200.5 100.5) (end 203.345 103.345) (width 0.5) (layer "F.Cu") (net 34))
 (segment (start 188.105 55.87) (end 181.285 62.69) (width 0.5) (layer "B.Cu") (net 23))
 (segment (start 181.285 62.69) (end 181.19 62.69) (width 0.5) (layer "B.Cu") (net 23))
 (segment (start 166.5 105) (end 166.5 99.08) (width 0.5) (layer "B.Cu") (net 43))
 (segment (start 193.185 104.13) (end 191.315 106) (width 0.5) (layer "B.Cu") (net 43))
 (segment (start 167.5 106) (end 166.5 105) (width 0.5) (layer "B.Cu") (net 43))
 (segment (start 191.315 106) (end 167.5 106) (width 0.5) (layer "B.Cu") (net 43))
 (segment (start 166.5 99.08) (end 165.5 98.08) (width 0.5) (layer "B.Cu") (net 43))
 (segment (start 170.295 62) (end 176.425 55.87) (width 0.5) (layer "B.Cu") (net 36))
 (segment (start 154.08 62) (end 170.295 62) (width 0.5) (layer "B.Cu") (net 36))
 (segment (start 164 76.19) (end 164 70.835) (width 0.5) (layer "F.Cu") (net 41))
 (segment (start 164 70.835) (end 178.965 55.87) (width 0.5) (layer "F.Cu") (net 41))
 (segment (start 163.81 76.19) (end 163.5 76.5) (width 0.5) (layer "B.Cu") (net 41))
 (segment (start 161.5 70.5) (end 168 64) (width 0.5) (layer "B.Cu") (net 10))
 (segment (start 168 64) (end 170.175405 64) (width 0.5) (layer "B.Cu") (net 10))
 (segment (start 175.675405 58.5) (end 179 58.5) (width 0.5) (layer "B.Cu") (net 10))
 (segment (start 179 58.375) (end 179 58.5) (width 0.5) (layer "B.Cu") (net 10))
 (segment (start 161.5 71.81) (end 161.5 70.5) (width 0.5) (layer "B.Cu") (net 10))
 (segment (start 181.505 55.87) (end 179 58.375) (width 0.5) (layer "B.Cu") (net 10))
 (segment (start 170.175405 64) (end 175.675405 58.5) (width 0.5) (layer "B.Cu") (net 10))
 (segment (start 200.805 56.195) (end 200.5 56.5) (width 0.5) (layer "B.Cu") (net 50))
 (segment (start 200.805 56.195) (end 200.805 55.87) (width 0.5) (layer "B.Cu") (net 50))
 (segment (start 200.805 101.805) (end 200.805 104.13) (width 0.5) (layer "F.Cu") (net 33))
 (segment (start 205 86.2) (end 199.5 91.7) (width 0.5) (layer "F.Cu") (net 33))
 (segment (start 199.5 100.5) (end 200.805 101.805) (width 0.5) (layer "F.Cu") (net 33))
 (segment (start 199.5 91.7) (end 199.5 100.5) (width 0.5) (layer "F.Cu") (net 33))
 (segment (start 178.915 61) (end 175.5 61) (width 0.5) (layer "B.Cu") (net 26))
 (segment (start 175.5 61) (end 156.19 80.31) (width 0.5) (layer "B.Cu") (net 26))
 (segment (start 156.19 80.31) (end 152 80.31) (width 0.5) (layer "B.Cu") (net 26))
 (segment (start 152 80.31) (end 151.5 79.81) (width 0.5) (layer "B.Cu") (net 26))
 (segment (start 184.045 55.87) (end 178.915 61) (width 0.5) (layer "B.Cu") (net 26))
 (segment (start 193.185 58.315) (end 188.81 62.69) (width 0.5) (layer "B.Cu") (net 21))
 (segment (start 193.185 55.87) (end 193.185 58.315) (width 0.5) (layer "B.Cu") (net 21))
 (segment (start 145.5 72.5) (end 146.436 71.564) (width 0.5) (layer "F.Cu") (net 40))
 (segment (start 162.5 58.5) (end 171 58.5) (width 0.5) (layer "F.Cu") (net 40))
 (segment (start 171.345 58.155) (end 171.345 55.87) (width 0.5) (layer "F.Cu") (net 40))
 (segment (start 146.436 71.564) (end 149.436 71.564) (width 0.5) (layer "F.Cu") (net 40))
 (segment (start 171 58.5) (end 171.345 58.155) (width 0.5) (layer "F.Cu") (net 40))
 (segment (start 149.436 71.564) (end 162.5 58.5) (width 0.5) (layer "F.Cu") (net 40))
 (segment (start 198.265 104.13) (end 198.265 90.395) (width 0.5) (layer "F.Cu") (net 32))
 (segment (start 198.265 90.395) (end 205 83.66) (width 0.5) (layer "F.Cu") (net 32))
 (segment (start 190.645 55.87) (end 190.645 58.315) (width 0.5) (layer "B.Cu") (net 22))
 (segment (start 190.645 58.315) (end 186.27 62.69) (width 0.5) (layer "B.Cu") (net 22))
 (segment (start 195.725 55.87) (end 195.725 63.225) (width 0.5) (layer "F.Cu") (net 31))
 (segment (start 202 78.12) (end 205 81.12) (width 0.5) (layer "F.Cu") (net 31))
 (segment (start 202 69.5) (end 202 78.12) (width 0.5) (layer "F.Cu") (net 31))
 (segment (start 195.725 63.225) (end 202 69.5) (width 0.5) (layer "F.Cu") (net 31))
 (segment (start 203.345 55.87) (end 201 58.215) (width 0.5) (layer "B.Cu") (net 29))
 (segment (start 201 58.215) (end 201 72.04) (width 0.5) (layer "B.Cu") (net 29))
 (segment (start 201 72.04) (end 205 76.04) (width 0.5) (layer "B.Cu") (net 29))
 (segment (start 145.5 81) (end 145.5 77.58) (width 0.5) (layer "F.Cu") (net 25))
 (segment (start 151.5 87) (end 145.5 81) (width 0.5) (layer "F.Cu") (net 25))
 (via (at 151.5 87) (size 0.8) (drill 0.4) (layers "F.Cu" "B.Cu") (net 25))
 (segment (start 180.13 104.13) (end 178.753874 102.753874) (width 0.5) (layer "B.Cu") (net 25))
 (segment (start 157.5 93) (end 165.5 93) (width 0.5) (layer "B.Cu") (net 25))
 (segment (start 176.11 62.69) (end 166.5 72.3) (width 0.5) (layer "B.Cu") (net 25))
 (segment (start 166.5 72.3) (end 166.5 92) (width 0.5) (layer "B.Cu") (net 25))
 (segment (start 180.485 104.13) (end 180.13 104.13) (width 0.5) (layer "B.Cu") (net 25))
 (segment (start 171 98.5) (end 165.5 93) (width 0.5) (layer "B.Cu") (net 25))
 (segment (start 151.5 87) (end 157.5 93) (width 0.5) (layer "B.Cu") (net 25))
 (segment (start 166.5 92) (end 165.5 93) (width 0.5) (layer "B.Cu") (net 25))
 (segment (start 178.753874 102.753874) (end 171 102.753874) (width 0.5) (layer "B.Cu") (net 25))
 (segment (start 171 102.753874) (end 171 98.5) (width 0.5) (layer "B.Cu") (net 25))
 (segment (start 207 68.5) (end 207 78.58) (width 0.5) (layer "F.Cu") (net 30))
 (segment (start 198.265 55.87) (end 198.265 59.765) (width 0.5) (layer "F.Cu") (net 30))
 (segment (start 207 78.58) (end 205 78.58) (width 0.5) (layer "F.Cu") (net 30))
 (segment (start 198.265 59.765) (end 207 68.5) (width 0.5) (layer "F.Cu") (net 30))
 (segment (start 205.885 102) (end 205.885 104.13) (width 0.5) (layer "F.Cu") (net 35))
 (segment (start 205 102) (end 205.885 102) (width 0.5) (layer "F.Cu") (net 35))
 (segment (start 205 91.28) (end 205 102) (width 0.5) (layer "F.Cu") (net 35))
 (segment (start 148.5 102.58) (end 164 87.08) (width 0.5) (layer "F.Cu") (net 42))
 (segment (start 164 87.08) (end 164 83.81) (width 0.5) (layer "F.Cu") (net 42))
 (segment (start 157.69 68) (end 161.5 64.19) (width 0.5) (layer "F.Cu") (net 11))
 (segment (start 157 91.54) (end 157 68.5) (width 0.5) (layer "F.Cu") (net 11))
 (segment (start 157.5 68) (end 157.69 68) (width 0.5) (layer "F.Cu") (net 11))
 (segment (start 157 68.5) (end 157.5 68) (width 0.5) (layer "F.Cu") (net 11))
 (segment (start 148.5 100.04) (end 157 91.54) (width 0.5) (layer "F.Cu") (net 11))
 (segment (start 148.81 72.19) (end 148.5 72.5) (width 0.5) (layer "B.Cu") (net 27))
 (segment (start 148.5 72.5) (end 148.5 95.5) (width 0.5) (layer "B.Cu") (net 27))
 (segment (start 151.5 72.19) (end 148.81 72.19) (width 0.5) (layer "B.Cu") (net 27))
 (segment (start 196.5 74.74) (end 194.74 76.5) (width 0.5) (layer "F.Cu") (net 24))
 (segment (start 178.65 62.69) (end 182.96 67) (width 0.5) (layer "F.Cu") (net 24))
 (segment (start 182.96 67) (end 196.5 67) (width 0.5) (layer "F.Cu") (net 24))
 (segment (start 196.5 67) (end 196.5 74.74) (width 0.5) (layer "F.Cu") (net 24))
 (segment (start 186.27 75.65) (end 187.12 76.5) (width 0.5) (layer "B.Cu") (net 16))
 (segment (start 186.27 70.31) (end 186.27 75.65) (width 0.5) (layer "B.Cu") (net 16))
 (segment (start 183.73 75.65) (end 184.58 76.5) (width 0.5) (layer "B.Cu") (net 15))
 (segment (start 183.73 70.31) (end 183.73 75.65) (width 0.5) (layer "B.Cu") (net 15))
 (segment (start 191.35 70.31) (end 191.35 75.65) (width 0.5) (layer "B.Cu") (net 18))
 (segment (start 191.35 75.65) (end 192.2 76.5) (width 0.5) (layer "B.Cu") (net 18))
 (segment (start 181.19 75.65) (end 182.04 76.5) (width 0.5) (layer "B.Cu") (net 14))
 (segment (start 181.19 70.31) (end 181.19 75.65) (width 0.5) (layer "B.Cu") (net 14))
 (segment (start 178.65 75.65) (end 179.5 76.5) (width 0.5) (layer "B.Cu") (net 13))
 (segment (start 178.65 70.31) (end 178.65 75.65) (width 0.5) (layer "B.Cu") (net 13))
 (segment (start 188.81 70.31) (end 188.81 75.65) (width 0.5) (layer "B.Cu") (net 17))
 (segment (start 188.81 75.65) (end 189.66 76.5) (width 0.5) (layer "B.Cu") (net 17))
 (segment (start 176.11 70.31) (end 176.11 75.65) (width 0.5) (layer "B.Cu") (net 12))
 (segment (start 176.11 75.65) (end 176.96 76.5) (width 0.5) (layer "B.Cu") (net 12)))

